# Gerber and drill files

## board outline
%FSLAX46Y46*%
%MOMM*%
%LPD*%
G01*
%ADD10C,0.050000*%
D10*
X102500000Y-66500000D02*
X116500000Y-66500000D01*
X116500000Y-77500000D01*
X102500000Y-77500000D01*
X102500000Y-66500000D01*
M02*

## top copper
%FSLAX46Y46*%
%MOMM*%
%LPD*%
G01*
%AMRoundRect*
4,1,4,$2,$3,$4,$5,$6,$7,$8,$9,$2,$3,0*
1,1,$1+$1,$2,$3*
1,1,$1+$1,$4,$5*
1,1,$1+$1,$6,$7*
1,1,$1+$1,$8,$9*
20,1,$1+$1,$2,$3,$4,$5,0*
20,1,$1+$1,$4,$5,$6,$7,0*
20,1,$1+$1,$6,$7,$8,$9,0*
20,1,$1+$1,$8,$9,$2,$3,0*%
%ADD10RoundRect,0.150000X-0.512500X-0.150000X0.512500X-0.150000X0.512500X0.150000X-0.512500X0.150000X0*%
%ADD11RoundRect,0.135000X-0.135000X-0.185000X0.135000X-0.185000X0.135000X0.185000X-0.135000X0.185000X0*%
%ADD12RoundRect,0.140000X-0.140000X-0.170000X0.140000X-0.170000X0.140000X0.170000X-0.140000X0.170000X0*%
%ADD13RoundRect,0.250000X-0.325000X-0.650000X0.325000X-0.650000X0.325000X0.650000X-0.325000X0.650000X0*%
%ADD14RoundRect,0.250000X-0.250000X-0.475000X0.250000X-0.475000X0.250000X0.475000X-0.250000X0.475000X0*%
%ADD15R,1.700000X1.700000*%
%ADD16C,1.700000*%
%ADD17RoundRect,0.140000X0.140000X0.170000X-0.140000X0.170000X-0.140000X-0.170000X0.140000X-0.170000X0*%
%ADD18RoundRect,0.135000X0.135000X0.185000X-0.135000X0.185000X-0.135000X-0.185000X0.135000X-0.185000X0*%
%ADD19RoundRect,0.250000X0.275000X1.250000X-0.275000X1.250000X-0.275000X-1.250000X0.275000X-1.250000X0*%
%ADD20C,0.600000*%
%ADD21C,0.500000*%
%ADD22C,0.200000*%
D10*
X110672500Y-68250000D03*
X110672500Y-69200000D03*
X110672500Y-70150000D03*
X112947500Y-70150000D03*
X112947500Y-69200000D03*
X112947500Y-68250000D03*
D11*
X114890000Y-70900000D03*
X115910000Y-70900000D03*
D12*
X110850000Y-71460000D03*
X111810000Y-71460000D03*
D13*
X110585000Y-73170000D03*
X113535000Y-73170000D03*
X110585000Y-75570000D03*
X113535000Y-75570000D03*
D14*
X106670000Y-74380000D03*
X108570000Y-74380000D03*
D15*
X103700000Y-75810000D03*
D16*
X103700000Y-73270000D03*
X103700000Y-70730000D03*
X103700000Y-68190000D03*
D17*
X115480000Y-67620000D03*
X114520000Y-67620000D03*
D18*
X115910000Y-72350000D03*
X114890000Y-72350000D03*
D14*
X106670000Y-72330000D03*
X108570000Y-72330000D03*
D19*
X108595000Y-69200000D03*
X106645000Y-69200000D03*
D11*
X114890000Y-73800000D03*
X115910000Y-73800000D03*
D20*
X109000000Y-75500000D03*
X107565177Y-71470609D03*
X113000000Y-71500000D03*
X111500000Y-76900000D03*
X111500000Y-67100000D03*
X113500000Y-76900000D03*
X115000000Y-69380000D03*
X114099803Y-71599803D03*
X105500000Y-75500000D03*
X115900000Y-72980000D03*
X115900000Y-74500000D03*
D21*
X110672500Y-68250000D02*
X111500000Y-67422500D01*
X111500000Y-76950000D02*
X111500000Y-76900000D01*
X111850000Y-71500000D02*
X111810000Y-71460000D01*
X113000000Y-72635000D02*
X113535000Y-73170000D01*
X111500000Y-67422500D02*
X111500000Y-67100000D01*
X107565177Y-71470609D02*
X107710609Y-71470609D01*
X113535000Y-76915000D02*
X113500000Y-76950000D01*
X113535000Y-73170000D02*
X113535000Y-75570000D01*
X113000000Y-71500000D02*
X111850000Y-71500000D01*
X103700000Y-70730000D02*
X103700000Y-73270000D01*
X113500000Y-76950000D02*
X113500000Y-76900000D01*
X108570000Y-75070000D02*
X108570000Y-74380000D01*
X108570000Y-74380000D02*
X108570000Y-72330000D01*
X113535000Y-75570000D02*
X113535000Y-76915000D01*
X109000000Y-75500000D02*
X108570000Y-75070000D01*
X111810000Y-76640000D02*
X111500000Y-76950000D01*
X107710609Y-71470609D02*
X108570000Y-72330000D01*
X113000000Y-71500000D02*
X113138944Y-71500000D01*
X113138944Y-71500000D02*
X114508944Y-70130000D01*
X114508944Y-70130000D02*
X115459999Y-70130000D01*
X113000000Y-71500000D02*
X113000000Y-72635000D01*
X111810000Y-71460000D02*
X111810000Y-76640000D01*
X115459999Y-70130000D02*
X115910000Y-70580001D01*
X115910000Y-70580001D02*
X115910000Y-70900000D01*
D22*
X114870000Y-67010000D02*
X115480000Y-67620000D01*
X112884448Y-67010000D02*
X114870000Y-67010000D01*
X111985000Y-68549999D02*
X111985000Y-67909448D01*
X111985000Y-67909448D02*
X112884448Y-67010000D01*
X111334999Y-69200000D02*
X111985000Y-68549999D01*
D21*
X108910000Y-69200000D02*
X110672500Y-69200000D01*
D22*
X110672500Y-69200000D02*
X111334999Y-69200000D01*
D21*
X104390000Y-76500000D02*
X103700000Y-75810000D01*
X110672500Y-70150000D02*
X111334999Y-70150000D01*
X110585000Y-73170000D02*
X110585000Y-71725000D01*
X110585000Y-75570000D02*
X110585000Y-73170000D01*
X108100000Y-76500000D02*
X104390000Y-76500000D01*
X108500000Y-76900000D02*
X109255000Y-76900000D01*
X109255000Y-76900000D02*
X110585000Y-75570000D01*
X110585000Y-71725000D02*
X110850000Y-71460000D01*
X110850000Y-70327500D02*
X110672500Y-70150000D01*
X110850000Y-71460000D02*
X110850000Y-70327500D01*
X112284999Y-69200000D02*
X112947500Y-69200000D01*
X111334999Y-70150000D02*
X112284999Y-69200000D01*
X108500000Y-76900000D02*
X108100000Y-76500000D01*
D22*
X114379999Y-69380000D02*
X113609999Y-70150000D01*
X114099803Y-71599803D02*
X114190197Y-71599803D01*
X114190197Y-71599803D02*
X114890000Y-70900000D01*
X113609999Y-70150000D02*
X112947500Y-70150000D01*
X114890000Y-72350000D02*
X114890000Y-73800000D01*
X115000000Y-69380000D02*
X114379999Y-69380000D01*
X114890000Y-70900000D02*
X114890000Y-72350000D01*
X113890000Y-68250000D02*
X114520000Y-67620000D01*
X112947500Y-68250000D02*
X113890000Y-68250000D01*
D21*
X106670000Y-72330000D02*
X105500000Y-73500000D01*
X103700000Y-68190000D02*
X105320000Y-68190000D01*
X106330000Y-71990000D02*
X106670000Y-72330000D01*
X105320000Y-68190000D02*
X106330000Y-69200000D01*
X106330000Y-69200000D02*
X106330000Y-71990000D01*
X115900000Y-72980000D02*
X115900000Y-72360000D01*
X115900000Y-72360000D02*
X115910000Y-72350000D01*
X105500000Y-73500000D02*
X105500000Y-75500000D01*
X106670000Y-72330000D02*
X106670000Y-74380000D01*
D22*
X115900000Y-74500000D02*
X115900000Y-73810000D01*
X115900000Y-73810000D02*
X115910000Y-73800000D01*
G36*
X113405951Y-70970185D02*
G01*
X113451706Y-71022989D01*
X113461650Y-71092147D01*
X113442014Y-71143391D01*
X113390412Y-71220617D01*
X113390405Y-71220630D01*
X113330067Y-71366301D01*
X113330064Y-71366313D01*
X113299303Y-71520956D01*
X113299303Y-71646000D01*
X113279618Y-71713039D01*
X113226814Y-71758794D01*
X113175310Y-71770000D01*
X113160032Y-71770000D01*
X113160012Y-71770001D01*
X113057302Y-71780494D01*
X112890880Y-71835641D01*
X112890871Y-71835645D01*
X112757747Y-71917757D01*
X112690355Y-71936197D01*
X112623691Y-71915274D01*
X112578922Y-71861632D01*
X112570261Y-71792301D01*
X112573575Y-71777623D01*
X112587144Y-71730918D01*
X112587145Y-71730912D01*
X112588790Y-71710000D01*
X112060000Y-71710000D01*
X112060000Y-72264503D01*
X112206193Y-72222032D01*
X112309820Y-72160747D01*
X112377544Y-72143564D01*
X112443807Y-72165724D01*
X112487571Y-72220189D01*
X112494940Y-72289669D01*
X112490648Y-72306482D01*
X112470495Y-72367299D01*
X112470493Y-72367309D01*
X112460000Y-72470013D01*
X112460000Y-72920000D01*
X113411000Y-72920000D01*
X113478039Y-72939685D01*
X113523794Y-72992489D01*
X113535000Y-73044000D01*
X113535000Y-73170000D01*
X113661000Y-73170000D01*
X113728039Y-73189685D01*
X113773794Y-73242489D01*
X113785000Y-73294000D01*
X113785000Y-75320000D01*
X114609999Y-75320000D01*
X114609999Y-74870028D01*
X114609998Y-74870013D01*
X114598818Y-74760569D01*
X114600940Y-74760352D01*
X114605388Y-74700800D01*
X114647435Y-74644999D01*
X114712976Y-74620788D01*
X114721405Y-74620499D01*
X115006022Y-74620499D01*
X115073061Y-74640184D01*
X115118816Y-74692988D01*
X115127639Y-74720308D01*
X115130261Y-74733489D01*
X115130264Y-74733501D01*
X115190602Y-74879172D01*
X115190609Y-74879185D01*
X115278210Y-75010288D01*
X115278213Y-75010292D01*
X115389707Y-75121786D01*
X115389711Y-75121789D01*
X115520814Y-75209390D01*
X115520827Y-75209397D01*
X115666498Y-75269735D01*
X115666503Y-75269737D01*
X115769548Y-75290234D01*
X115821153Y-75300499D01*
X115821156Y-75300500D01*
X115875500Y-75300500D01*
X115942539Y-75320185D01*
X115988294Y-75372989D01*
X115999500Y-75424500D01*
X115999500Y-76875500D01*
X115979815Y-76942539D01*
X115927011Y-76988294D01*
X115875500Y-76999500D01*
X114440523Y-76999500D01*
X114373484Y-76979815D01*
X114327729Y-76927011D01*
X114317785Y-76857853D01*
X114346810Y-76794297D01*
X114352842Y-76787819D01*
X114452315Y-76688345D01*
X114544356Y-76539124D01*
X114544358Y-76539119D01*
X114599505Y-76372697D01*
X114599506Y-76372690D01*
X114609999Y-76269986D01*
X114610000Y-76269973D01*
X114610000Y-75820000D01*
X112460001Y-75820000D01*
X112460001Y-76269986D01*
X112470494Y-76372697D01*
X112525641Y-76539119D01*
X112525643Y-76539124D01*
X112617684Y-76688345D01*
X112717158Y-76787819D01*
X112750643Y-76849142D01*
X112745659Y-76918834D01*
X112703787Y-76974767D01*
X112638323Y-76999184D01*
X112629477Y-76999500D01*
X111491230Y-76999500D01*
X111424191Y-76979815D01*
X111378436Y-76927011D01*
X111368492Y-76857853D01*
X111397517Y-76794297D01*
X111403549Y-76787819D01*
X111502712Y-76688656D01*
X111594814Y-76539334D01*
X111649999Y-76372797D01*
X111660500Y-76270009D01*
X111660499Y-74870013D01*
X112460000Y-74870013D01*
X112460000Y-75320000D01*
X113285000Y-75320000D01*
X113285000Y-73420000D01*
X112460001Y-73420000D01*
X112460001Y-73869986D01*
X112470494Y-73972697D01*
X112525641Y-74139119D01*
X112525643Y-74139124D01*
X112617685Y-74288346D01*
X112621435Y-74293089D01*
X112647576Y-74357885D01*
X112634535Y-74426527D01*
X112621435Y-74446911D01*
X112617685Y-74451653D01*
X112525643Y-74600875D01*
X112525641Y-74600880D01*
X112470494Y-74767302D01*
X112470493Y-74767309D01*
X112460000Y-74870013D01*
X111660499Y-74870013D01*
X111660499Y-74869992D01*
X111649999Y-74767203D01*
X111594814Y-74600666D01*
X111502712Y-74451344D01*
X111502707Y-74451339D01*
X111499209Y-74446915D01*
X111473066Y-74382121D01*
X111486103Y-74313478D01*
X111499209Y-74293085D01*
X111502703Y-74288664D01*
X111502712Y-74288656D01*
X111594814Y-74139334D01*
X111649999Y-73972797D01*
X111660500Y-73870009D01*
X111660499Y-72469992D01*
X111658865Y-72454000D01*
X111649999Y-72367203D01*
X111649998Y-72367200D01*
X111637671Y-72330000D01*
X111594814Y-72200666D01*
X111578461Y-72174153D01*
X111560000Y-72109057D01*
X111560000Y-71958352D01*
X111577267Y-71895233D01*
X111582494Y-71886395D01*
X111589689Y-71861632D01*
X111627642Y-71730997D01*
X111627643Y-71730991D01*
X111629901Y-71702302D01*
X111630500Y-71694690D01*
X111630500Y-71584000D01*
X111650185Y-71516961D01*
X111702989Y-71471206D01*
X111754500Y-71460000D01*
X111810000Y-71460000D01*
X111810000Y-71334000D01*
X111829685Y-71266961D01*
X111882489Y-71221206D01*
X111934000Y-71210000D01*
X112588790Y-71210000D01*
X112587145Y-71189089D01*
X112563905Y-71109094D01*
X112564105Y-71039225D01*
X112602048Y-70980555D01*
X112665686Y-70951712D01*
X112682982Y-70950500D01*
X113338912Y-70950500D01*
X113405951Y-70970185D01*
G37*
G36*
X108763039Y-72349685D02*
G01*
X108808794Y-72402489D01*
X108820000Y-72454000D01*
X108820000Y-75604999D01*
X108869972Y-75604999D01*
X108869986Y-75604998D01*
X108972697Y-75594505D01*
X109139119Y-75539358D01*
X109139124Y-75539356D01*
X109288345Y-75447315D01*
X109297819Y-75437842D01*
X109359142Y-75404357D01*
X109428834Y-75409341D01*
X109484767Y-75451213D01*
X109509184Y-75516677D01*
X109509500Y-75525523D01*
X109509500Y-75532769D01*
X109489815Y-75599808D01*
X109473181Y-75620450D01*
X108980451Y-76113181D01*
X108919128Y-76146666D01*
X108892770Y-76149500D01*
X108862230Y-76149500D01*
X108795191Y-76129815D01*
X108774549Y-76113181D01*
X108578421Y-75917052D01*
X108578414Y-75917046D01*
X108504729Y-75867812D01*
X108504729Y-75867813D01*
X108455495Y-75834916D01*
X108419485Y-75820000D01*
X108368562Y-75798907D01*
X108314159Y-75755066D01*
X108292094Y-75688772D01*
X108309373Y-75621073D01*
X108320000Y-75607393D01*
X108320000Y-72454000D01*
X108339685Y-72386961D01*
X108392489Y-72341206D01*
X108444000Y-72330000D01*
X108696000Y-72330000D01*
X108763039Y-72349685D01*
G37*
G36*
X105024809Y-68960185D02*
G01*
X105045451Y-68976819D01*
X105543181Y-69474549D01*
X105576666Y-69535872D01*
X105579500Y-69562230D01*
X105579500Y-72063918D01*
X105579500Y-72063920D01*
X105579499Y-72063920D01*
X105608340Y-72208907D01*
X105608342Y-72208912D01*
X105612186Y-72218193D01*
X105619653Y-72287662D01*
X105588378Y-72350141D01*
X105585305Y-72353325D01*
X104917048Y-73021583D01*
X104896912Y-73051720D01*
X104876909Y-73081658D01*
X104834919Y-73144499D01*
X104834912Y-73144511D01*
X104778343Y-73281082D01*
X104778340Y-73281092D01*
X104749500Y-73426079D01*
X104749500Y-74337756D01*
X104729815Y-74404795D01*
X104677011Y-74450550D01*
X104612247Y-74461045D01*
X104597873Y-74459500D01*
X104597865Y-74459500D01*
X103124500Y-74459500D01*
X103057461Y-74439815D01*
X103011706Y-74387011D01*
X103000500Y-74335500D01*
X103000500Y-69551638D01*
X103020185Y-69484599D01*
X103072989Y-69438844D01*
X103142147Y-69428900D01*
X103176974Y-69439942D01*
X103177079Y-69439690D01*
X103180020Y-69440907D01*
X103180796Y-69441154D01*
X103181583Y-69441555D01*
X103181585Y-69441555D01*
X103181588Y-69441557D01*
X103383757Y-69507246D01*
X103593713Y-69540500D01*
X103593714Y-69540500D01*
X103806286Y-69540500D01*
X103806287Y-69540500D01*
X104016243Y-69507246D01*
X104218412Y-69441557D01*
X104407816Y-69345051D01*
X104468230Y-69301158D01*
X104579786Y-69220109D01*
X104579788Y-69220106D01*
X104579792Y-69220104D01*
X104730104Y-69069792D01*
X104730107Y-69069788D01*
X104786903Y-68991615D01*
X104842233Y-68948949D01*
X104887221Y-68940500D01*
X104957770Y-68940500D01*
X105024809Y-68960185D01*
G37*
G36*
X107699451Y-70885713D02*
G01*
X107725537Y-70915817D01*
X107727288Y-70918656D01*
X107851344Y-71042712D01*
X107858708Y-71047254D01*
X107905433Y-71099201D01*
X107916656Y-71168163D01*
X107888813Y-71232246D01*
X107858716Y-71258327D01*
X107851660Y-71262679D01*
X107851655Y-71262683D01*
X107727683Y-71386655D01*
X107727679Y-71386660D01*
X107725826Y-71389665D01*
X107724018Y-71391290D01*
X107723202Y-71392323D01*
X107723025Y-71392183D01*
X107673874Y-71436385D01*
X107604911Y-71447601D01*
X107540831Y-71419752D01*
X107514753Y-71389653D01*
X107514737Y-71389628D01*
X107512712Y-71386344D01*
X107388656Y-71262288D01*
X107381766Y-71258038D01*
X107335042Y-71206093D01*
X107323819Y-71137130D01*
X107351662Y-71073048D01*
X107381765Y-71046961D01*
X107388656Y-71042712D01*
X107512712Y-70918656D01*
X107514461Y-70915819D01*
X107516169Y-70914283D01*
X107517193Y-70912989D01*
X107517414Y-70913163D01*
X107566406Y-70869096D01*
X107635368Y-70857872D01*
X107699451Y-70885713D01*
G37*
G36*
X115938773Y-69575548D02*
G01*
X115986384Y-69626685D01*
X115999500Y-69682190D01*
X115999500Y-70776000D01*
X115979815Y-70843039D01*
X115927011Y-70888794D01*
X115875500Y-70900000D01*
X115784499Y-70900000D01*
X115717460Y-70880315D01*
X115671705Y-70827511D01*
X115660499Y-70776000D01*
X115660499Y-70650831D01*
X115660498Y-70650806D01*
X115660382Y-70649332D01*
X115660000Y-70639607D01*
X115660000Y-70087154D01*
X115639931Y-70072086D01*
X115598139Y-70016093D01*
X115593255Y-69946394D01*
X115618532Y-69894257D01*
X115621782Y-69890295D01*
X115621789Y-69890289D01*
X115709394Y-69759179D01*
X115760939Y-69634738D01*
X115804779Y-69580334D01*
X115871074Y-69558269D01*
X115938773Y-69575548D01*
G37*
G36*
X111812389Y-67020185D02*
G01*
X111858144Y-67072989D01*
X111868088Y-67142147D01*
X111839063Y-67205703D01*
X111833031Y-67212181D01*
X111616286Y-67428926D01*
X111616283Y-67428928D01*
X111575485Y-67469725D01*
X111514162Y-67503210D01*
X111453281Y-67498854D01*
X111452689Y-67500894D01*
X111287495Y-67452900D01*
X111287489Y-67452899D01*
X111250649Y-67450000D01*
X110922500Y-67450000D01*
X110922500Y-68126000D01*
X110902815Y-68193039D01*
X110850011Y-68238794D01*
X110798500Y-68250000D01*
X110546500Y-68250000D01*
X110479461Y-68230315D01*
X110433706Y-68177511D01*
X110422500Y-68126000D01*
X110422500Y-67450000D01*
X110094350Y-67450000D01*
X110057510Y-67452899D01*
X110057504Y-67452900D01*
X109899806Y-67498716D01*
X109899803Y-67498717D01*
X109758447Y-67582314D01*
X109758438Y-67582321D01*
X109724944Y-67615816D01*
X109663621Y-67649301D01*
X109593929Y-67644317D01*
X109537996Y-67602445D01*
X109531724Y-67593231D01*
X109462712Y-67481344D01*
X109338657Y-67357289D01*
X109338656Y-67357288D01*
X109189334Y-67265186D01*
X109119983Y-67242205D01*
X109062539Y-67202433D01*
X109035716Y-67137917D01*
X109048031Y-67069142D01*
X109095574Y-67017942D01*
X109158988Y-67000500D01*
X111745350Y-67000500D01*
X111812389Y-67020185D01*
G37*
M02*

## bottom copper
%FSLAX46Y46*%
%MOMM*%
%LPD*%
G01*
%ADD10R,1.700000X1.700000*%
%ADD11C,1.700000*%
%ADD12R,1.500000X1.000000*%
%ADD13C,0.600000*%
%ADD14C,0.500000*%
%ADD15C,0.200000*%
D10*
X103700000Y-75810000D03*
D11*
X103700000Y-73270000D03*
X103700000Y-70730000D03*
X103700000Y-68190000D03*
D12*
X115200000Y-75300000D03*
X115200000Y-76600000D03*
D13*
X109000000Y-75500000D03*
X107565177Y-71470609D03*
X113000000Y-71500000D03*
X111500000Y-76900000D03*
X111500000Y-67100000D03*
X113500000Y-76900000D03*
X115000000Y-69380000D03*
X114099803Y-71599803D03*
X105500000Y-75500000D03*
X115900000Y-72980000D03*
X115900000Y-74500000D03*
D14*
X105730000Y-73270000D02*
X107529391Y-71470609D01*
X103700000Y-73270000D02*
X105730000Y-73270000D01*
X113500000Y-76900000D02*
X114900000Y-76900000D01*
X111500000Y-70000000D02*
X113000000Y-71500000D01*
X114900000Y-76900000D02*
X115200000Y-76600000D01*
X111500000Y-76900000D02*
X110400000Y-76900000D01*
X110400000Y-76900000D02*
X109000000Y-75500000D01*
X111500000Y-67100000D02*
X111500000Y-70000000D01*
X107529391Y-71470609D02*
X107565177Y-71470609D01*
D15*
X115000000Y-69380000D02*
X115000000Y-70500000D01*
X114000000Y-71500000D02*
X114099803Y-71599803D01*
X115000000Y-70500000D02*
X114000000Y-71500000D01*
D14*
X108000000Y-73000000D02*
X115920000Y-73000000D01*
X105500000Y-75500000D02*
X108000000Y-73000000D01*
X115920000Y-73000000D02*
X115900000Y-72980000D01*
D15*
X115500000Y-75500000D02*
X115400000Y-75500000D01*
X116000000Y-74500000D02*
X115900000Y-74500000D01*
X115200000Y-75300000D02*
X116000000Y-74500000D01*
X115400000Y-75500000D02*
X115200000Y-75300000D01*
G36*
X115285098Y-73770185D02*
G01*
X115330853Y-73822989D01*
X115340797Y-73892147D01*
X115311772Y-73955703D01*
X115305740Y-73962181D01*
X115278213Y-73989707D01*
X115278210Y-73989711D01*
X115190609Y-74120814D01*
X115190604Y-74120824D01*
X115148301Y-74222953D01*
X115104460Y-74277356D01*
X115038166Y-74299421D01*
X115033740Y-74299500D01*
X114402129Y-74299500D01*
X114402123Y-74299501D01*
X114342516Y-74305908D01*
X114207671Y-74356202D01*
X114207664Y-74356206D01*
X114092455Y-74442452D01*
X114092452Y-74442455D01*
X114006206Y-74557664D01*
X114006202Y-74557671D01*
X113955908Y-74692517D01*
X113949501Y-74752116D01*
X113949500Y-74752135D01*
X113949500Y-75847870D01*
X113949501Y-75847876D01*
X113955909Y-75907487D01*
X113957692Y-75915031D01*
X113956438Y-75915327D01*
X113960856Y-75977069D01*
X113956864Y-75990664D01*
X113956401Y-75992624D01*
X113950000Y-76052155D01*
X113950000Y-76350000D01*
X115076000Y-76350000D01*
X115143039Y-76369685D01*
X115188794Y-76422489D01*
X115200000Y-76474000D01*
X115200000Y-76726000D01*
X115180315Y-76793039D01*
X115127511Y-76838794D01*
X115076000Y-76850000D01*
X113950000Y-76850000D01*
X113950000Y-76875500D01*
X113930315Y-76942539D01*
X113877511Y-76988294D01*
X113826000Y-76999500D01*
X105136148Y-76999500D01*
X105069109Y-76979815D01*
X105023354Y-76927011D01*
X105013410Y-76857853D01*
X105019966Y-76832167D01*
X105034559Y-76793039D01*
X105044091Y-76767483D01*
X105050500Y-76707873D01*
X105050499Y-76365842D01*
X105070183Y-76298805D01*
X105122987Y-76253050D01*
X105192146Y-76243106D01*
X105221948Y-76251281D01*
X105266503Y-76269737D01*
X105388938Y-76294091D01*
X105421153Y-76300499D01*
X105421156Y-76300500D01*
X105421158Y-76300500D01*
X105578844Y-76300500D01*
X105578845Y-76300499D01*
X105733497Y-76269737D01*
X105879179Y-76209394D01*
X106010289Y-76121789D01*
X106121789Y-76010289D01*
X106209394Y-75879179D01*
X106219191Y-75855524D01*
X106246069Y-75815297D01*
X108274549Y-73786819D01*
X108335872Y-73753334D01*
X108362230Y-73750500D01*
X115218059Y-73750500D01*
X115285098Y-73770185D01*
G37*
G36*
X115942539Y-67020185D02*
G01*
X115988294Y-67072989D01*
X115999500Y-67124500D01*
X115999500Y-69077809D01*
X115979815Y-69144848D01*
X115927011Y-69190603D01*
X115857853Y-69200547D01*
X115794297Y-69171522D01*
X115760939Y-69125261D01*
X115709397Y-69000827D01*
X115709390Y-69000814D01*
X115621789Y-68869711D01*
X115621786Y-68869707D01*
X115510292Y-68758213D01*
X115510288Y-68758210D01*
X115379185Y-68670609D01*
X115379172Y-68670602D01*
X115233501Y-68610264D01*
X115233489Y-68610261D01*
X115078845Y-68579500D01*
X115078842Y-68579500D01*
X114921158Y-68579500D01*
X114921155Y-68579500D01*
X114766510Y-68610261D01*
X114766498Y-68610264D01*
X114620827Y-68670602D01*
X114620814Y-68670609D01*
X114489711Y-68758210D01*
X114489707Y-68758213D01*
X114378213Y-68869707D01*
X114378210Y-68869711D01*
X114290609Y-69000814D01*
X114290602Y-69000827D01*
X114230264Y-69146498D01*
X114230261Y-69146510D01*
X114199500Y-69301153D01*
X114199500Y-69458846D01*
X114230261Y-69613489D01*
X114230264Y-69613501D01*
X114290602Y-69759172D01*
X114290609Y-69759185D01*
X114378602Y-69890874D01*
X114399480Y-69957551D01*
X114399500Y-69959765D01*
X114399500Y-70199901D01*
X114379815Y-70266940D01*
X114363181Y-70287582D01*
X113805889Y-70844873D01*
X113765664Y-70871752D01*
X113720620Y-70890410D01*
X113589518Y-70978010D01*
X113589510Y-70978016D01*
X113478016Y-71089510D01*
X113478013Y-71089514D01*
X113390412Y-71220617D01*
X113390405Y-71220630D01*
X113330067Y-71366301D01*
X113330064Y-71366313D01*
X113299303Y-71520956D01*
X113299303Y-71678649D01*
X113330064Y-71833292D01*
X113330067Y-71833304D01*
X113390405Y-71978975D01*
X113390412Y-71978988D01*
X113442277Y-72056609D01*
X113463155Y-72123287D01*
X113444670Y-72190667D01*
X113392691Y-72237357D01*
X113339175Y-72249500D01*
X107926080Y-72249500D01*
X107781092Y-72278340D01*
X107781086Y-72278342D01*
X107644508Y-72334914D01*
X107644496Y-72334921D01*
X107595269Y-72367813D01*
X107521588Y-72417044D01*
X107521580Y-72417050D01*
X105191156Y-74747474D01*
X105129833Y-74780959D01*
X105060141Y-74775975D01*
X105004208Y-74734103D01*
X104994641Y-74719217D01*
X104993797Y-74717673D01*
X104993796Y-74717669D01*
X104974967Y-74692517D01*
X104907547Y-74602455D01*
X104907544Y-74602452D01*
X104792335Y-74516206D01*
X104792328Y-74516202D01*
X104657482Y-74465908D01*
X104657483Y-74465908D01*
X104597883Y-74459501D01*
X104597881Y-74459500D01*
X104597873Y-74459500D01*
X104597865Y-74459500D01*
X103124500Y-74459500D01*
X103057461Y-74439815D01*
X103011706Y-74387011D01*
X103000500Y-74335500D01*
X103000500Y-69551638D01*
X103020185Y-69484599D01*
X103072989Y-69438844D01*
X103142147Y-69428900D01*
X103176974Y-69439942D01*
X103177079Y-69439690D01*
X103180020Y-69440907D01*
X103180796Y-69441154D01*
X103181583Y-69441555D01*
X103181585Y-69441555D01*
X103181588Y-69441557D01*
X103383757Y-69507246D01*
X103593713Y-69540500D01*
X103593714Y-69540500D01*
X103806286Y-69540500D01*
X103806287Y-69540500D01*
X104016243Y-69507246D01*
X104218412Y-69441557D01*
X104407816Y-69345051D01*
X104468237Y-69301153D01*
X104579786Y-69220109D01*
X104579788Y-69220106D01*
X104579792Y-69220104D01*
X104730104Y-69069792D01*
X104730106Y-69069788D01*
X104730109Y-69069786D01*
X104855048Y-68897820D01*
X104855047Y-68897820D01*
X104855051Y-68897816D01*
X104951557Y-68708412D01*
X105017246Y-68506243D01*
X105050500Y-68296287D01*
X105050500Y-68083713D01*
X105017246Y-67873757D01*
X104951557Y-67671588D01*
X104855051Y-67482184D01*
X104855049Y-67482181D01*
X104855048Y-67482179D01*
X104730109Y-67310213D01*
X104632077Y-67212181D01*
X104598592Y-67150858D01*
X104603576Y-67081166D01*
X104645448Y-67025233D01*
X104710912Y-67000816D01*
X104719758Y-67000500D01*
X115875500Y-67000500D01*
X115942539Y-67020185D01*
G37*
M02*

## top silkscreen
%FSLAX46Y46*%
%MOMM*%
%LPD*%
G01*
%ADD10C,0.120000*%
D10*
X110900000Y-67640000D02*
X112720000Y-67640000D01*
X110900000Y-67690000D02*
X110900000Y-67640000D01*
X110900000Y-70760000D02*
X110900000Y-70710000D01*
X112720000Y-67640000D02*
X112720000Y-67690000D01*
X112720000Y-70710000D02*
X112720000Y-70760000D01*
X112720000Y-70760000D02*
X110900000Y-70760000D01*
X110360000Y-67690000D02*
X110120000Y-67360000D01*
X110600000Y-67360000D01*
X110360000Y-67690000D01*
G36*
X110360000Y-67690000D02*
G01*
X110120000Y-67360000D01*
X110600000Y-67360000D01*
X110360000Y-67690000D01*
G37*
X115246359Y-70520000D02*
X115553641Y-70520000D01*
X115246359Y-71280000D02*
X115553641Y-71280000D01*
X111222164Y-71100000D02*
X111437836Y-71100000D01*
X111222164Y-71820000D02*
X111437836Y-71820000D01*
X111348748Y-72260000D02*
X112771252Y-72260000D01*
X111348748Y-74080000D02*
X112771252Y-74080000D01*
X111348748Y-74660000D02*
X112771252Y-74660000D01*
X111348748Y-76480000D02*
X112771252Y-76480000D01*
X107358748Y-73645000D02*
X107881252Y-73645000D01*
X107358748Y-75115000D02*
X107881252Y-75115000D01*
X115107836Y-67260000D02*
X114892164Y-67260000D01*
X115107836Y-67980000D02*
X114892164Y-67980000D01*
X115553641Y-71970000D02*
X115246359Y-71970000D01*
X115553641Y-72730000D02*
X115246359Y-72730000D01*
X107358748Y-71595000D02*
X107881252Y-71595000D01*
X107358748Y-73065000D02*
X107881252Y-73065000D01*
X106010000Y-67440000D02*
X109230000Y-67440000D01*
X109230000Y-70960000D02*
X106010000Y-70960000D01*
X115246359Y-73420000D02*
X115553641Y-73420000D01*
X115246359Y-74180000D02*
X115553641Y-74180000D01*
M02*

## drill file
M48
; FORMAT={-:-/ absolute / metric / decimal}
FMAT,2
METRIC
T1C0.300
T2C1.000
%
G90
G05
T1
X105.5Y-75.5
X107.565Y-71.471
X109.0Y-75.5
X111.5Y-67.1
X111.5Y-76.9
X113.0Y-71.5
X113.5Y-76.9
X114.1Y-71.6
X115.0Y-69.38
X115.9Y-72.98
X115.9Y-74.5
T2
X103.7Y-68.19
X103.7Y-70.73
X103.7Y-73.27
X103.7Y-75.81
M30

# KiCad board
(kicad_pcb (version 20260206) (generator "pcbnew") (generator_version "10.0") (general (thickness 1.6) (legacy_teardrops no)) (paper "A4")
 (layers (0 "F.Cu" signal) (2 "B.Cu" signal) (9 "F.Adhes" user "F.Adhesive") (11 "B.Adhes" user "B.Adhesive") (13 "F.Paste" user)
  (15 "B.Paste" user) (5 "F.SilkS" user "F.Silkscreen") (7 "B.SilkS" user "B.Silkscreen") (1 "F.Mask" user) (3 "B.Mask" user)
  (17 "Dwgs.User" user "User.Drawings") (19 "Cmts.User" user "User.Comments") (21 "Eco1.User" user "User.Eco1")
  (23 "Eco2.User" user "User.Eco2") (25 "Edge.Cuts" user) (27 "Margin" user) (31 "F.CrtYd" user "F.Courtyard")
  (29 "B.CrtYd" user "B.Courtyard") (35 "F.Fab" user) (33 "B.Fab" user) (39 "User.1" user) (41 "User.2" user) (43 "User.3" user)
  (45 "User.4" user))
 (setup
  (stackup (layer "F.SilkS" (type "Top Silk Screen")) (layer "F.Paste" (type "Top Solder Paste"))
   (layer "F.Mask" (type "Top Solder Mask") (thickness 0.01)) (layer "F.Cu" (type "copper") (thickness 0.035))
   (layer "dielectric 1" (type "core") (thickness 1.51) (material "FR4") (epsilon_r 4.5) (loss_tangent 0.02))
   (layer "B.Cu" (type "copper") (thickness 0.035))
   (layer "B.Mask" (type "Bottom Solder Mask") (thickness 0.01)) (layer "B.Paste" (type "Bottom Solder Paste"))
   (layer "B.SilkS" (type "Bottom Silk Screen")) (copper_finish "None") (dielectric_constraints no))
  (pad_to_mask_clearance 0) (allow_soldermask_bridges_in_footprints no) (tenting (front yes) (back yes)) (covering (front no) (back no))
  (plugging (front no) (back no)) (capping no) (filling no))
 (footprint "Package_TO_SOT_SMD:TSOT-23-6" (layer "F.Cu") (at 111.81 69.2)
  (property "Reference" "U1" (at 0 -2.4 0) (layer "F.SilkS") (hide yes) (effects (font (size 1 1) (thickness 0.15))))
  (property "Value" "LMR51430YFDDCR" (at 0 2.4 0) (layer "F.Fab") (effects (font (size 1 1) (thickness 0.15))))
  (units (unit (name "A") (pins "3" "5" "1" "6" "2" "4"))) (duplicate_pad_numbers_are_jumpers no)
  (fp_line (start -0.91 -1.56) (end 0.91 -1.56) (stroke (width 0.12) (type solid)) (layer "F.SilkS"))
  (fp_line (start -0.91 -1.51) (end -0.91 -1.56) (stroke (width 0.12) (type solid)) (layer "F.SilkS"))
  (fp_line (start -0.91 1.56) (end -0.91 1.51) (stroke (width 0.12) (type solid)) (layer "F.SilkS"))
  (fp_line (start 0.91 -1.56) (end 0.91 -1.51) (stroke (width 0.12) (type solid)) (layer "F.SilkS"))
  (fp_line (start 0.91 1.51) (end 0.91 1.56) (stroke (width 0.12) (type solid)) (layer "F.SilkS"))
  (fp_line (start 0.91 1.56) (end -0.91 1.56) (stroke (width 0.12) (type solid)) (layer "F.SilkS"))
  (fp_poly (pts (xy -1.45 -1.51) (xy -1.69 -1.84) (xy -1.21 -1.84)) (stroke (width 0.12) (type solid)) (fill yes) (layer "F.SilkS"))
  (pad "1" smd roundrect (at -1.1375 -0.95) (size 1.325 0.6) (layers "F.Cu" "F.Mask" "F.Paste") (roundrect_rratio 0.25) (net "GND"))
  (pad "2" smd roundrect (at -1.1375 0) (size 1.325 0.6) (layers "F.Cu" "F.Mask" "F.Paste") (roundrect_rratio 0.25) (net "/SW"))
  (pad "3" smd roundrect (at -1.1375 0.95) (size 1.325 0.6) (layers "F.Cu" "F.Mask" "F.Paste") (roundrect_rratio 0.25) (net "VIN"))
  (pad "4" smd roundrect (at 1.1375 0.95) (size 1.325 0.6) (layers "F.Cu" "F.Mask" "F.Paste") (roundrect_rratio 0.25) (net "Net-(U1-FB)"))
  (pad "5" smd roundrect (at 1.1375 0) (size 1.325 0.6) (layers "F.Cu" "F.Mask" "F.Paste") (roundrect_rratio 0.25) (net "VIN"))
  (pad "6" smd roundrect (at 1.1375 -0.95) (size 1.325 0.6) (layers "F.Cu" "F.Mask" "F.Paste") (roundrect_rratio 0.25) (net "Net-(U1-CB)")))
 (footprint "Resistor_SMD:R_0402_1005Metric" (layer "F.Cu") (at 115.4 70.9)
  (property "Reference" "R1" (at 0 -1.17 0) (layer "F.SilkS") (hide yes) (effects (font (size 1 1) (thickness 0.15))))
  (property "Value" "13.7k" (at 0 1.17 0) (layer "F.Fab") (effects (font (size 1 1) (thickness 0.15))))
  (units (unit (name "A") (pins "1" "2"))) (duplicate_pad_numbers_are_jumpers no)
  (fp_line (start -0.153641 -0.38) (end 0.153641 -0.38) (stroke (width 0.12) (type solid)) (layer "F.SilkS"))
  (fp_line (start -0.153641 0.38) (end 0.153641 0.38) (stroke (width 0.12) (type solid)) (layer "F.SilkS"))
  (pad "1" smd roundrect (at -0.51 0) (size 0.54 0.64) (layers "F.Cu" "F.Mask" "F.Paste") (roundrect_rratio 0.25) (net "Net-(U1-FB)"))
  (pad "2" smd roundrect (at 0.51 0) (size 0.54 0.64) (layers "F.Cu" "F.Mask" "F.Paste") (roundrect_rratio 0.25) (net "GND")))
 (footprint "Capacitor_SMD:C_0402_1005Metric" (layer "F.Cu") (at 111.33 71.46)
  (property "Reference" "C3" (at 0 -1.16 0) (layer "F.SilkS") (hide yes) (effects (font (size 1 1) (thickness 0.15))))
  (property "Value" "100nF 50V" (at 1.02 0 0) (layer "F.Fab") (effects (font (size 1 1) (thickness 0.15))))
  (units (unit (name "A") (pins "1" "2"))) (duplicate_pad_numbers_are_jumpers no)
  (fp_line (start -0.107836 -0.36) (end 0.107836 -0.36) (stroke (width 0.12) (type solid)) (layer "F.SilkS"))
  (fp_line (start -0.107836 0.36) (end 0.107836 0.36) (stroke (width 0.12) (type solid)) (layer "F.SilkS"))
  (pad "1" smd roundrect (at -0.48 0) (size 0.56 0.62) (layers "F.Cu" "F.Mask" "F.Paste") (roundrect_rratio 0.25) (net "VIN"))
  (pad "2" smd roundrect (at 0.48 0) (size 0.56 0.62) (layers "F.Cu" "F.Mask" "F.Paste") (roundrect_rratio 0.25) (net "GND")))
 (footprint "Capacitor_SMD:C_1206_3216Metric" (layer "F.Cu") (at 112.06 73.17)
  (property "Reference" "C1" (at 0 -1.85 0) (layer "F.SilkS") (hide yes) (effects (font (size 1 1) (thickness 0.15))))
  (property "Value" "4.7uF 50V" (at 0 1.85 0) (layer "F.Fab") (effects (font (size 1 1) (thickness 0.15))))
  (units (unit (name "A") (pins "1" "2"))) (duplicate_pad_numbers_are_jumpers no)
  (fp_line (start -0.711252 -0.91) (end 0.711252 -0.91) (stroke (width 0.12) (type solid)) (layer "F.SilkS"))
  (fp_line (start -0.711252 0.91) (end 0.711252 0.91) (stroke (width 0.12) (type solid)) (layer "F.SilkS"))
  (pad "1" smd roundrect (at -1.475 0) (size 1.15 1.8) (layers "F.Cu" "F.Mask" "F.Paste") (roundrect_rratio 0.217391) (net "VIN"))
  (pad "2" smd roundrect (at 1.475 0) (size 1.15 1.8) (layers "F.Cu" "F.Mask" "F.Paste") (roundrect_rratio 0.217391) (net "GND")))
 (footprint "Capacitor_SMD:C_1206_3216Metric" (layer "F.Cu") (at 112.06 75.57)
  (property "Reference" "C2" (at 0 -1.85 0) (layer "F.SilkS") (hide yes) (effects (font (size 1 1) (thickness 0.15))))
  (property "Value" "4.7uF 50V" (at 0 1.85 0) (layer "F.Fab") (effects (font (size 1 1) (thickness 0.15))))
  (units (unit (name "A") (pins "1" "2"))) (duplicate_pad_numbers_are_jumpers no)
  (fp_line (start -0.711252 -0.91) (end 0.711252 -0.91) (stroke (width 0.12) (type solid)) (layer "F.SilkS"))
  (fp_line (start -0.711252 0.91) (end 0.711252 0.91) (stroke (width 0.12) (type solid)) (layer "F.SilkS"))
  (pad "1" smd roundrect (at -1.475 0) (size 1.15 1.8) (layers "F.Cu" "F.Mask" "F.Paste") (roundrect_rratio 0.217391) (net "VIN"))
  (pad "2" smd roundrect (at 1.475 0) (size 1.15 1.8) (layers "F.Cu" "F.Mask" "F.Paste") (roundrect_rratio 0.217391) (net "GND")))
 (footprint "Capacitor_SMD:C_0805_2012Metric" (layer "F.Cu") (at 107.62 74.38)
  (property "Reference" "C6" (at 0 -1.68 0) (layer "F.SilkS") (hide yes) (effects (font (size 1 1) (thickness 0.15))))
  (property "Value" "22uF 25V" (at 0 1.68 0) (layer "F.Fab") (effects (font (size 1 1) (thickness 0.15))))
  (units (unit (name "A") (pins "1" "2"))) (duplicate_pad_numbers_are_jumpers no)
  (fp_line (start -0.261252 -0.735) (end 0.261252 -0.735) (stroke (width 0.12) (type solid)) (layer "F.SilkS"))
  (fp_line (start -0.261252 0.735) (end 0.261252 0.735) (stroke (width 0.12) (type solid)) (layer "F.SilkS"))
  (pad "1" smd roundrect (at -0.95 0) (size 1 1.45) (layers "F.Cu" "F.Mask" "F.Paste") (roundrect_rratio 0.25) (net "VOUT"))
  (pad "2" smd roundrect (at 0.95 0) (size 1 1.45) (layers "F.Cu" "F.Mask" "F.Paste") (roundrect_rratio 0.25) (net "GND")))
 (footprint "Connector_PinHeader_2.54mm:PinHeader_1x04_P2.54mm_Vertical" (layer "F.Cu") (at 103.7 75.81 180)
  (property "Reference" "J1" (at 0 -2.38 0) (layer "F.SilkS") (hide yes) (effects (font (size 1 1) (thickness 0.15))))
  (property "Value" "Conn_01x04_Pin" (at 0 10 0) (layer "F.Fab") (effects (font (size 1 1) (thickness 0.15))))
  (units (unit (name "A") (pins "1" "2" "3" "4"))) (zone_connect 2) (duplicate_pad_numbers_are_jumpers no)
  (pad "1" thru_hole rect (at 0 0 180) (size 1.7 1.7) (drill 1) (layers "*.Cu" "*.Mask") (remove_unused_layers no) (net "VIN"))
  (pad "2" thru_hole circle (at 0 2.54 180) (size 1.7 1.7) (drill 1) (layers "*.Cu" "*.Mask") (remove_unused_layers no) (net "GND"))
  (pad "3" thru_hole circle (at 0 5.08 180) (size 1.7 1.7) (drill 1) (layers "*.Cu" "*.Mask") (remove_unused_layers no) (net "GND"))
  (pad "4" thru_hole circle (at 0 7.62 180) (size 1.7 1.7) (drill 1) (layers "*.Cu" "*.Mask") (remove_unused_layers no) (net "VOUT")))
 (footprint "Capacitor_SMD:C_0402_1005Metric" (layer "F.Cu") (at 115 67.62 180)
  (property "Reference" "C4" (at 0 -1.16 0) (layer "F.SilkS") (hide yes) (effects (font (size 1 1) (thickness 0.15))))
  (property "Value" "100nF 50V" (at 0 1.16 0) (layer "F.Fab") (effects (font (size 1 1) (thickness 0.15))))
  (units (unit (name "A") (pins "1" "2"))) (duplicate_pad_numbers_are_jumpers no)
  (fp_line (start -0.107836 0.36) (end 0.107836 0.36) (stroke (width 0.12) (type solid)) (layer "F.SilkS"))
  (fp_line (start -0.107836 -0.36) (end 0.107836 -0.36) (stroke (width 0.12) (type solid)) (layer "F.SilkS"))
  (pad "1" smd roundrect (at -0.48 0 180) (size 0.56 0.62) (layers "F.Cu" "F.Mask" "F.Paste") (roundrect_rratio 0.25) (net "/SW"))
  (pad "2" smd roundrect (at 0.48 0 180) (size 0.56 0.62) (layers "F.Cu" "F.Mask" "F.Paste") (roundrect_rratio 0.25) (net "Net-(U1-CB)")))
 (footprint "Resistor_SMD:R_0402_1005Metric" (layer "F.Cu") (at 115.4 72.35 180)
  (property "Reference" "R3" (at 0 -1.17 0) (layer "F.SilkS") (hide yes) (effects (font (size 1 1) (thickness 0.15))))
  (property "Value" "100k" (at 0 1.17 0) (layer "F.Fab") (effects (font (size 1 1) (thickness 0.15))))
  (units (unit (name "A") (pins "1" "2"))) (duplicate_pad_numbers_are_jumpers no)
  (fp_line (start -0.153641 0.38) (end 0.153641 0.38) (stroke (width 0.12) (type solid)) (layer "F.SilkS"))
  (fp_line (start -0.153641 -0.38) (end 0.153641 -0.38) (stroke (width 0.12) (type solid)) (layer "F.SilkS"))
  (pad "1" smd roundrect (at -0.51 0 180) (size 0.54 0.64) (layers "F.Cu" "F.Mask" "F.Paste") (roundrect_rratio 0.25) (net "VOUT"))
  (pad "2" smd roundrect (at 0.51 0 180) (size 0.54 0.64) (layers "F.Cu" "F.Mask" "F.Paste") (roundrect_rratio 0.25) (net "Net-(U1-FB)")))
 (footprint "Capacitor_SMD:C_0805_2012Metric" (layer "F.Cu") (at 107.62 72.33)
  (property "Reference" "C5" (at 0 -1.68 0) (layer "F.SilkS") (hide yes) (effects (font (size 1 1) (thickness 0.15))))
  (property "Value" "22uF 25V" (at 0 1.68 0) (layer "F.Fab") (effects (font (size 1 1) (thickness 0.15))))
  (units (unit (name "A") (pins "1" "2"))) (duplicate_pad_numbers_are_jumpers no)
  (fp_line (start -0.261252 -0.735) (end 0.261252 -0.735) (stroke (width 0.12) (type solid)) (layer "F.SilkS"))
  (fp_line (start -0.261252 0.735) (end 0.261252 0.735) (stroke (width 0.12) (type solid)) (layer "F.SilkS"))
  (pad "1" smd roundrect (at -0.95 0) (size 1 1.45) (layers "F.Cu" "F.Mask" "F.Paste") (roundrect_rratio 0.25) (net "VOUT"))
  (pad "2" smd roundrect (at 0.95 0) (size 1 1.45) (layers "F.Cu" "F.Mask" "F.Paste") (roundrect_rratio 0.25) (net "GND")))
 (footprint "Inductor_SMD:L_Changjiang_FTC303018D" (layer "F.Cu") (at 107.62 69.2 180)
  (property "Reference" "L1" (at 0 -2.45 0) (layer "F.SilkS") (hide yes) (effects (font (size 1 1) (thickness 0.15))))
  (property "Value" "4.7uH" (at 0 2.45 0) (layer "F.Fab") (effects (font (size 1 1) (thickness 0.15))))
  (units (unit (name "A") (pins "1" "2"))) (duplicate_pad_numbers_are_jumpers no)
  (fp_line (start 1.61 1.76) (end -1.61 1.76) (stroke (width 0.12) (type solid)) (layer "F.SilkS"))
  (fp_line (start -1.61 -1.76) (end 1.61 -1.76) (stroke (width 0.12) (type solid)) (layer "F.SilkS"))
  (pad "1" smd roundrect (at -0.975 0 180) (size 1.05 3) (layers "F.Cu" "F.Mask" "F.Paste") (roundrect_rratio 0.238095) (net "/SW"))
  (pad "2" smd roundrect (at 0.975 0 180) (size 1.05 3) (layers "F.Cu" "F.Mask" "F.Paste") (roundrect_rratio 0.238095) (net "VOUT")))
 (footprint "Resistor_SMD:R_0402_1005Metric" (layer "F.Cu") (at 115.4 73.8)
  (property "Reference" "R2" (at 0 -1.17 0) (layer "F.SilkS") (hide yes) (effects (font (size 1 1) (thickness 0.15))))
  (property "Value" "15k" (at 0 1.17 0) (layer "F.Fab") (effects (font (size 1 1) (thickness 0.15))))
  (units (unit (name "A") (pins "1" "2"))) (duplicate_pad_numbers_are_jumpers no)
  (fp_line (start -0.153641 -0.38) (end 0.153641 -0.38) (stroke (width 0.12) (type solid)) (layer "F.SilkS"))
  (fp_line (start -0.153641 0.38) (end 0.153641 0.38) (stroke (width 0.12) (type solid)) (layer "F.SilkS"))
  (pad "1" smd roundrect (at -0.51 0) (size 0.54 0.64) (layers "F.Cu" "F.Mask" "F.Paste") (roundrect_rratio 0.25) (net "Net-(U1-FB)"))
  (pad "2" smd roundrect (at 0.51 0) (size 0.54 0.64) (layers "F.Cu" "F.Mask" "F.Paste") (roundrect_rratio 0.25) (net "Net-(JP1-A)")))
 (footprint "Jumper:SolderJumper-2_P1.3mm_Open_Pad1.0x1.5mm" (layer "B.Cu") (at 115.2 75.95 -90)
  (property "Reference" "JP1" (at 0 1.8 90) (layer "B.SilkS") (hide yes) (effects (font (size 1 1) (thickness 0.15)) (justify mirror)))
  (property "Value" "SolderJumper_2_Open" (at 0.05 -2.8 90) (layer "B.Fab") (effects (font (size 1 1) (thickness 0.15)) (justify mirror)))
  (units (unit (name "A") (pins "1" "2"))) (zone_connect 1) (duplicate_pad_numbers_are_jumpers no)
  (pad "1" smd rect (at -0.65 0 270) (size 1 1.5) (layers "B.Cu" "B.Mask") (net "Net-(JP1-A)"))
  (pad "2" smd rect (at 0.65 0 270) (size 1 1.5) (layers "B.Cu" "B.Mask") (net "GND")))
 (gr_rect (start 102.5 66.5) (end 116.5 77.5) (stroke (width 0.05) (type default)) (fill no) (layer "Edge.Cuts"))
 (segment (start 110.6725 68.25) (end 111.5 67.4225) (width 0.5) (layer "F.Cu") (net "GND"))
 (segment (start 111.5 76.95) (end 111.5 76.9) (width 0.5) (layer "F.Cu") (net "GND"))
 (segment (start 111.85 71.5) (end 111.81 71.46) (width 0.5) (layer "F.Cu") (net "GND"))
 (segment (start 113 72.635) (end 113.535 73.17) (width 0.5) (layer "F.Cu") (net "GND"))
 (segment (start 111.5 67.4225) (end 111.5 67.1) (width 0.5) (layer "F.Cu") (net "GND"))
 (segment (start 107.565177 71.470609) (end 107.710609 71.470609) (width 0.5) (layer "F.Cu") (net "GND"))
 (segment (start 113.535 76.915) (end 113.5 76.95) (width 0.5) (layer "F.Cu") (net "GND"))
 (segment (start 113.535 73.17) (end 113.535 75.57) (width 0.5) (layer "F.Cu") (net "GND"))
 (segment (start 113 71.5) (end 111.85 71.5) (width 0.5) (layer "F.Cu") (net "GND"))
 (segment (start 103.7 70.73) (end 103.7 73.27) (width 0.5) (layer "F.Cu") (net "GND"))
 (segment (start 113.5 76.95) (end 113.5 76.9) (width 0.5) (layer "F.Cu") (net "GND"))
 (segment (start 108.57 75.07) (end 108.57 74.38) (width 0.5) (layer "F.Cu") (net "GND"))
 (segment (start 108.57 74.38) (end 108.57 72.33) (width 0.5) (layer "F.Cu") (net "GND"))
 (segment (start 113.535 75.57) (end 113.535 76.915) (width 0.5) (layer "F.Cu") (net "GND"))
 (segment (start 109 75.5) (end 108.57 75.07) (width 0.5) (layer "F.Cu") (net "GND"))
 (segment (start 111.81 76.64) (end 111.5 76.95) (width 0.5) (layer "F.Cu") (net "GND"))
 (segment (start 107.710609 71.470609) (end 108.57 72.33) (width 0.5) (layer "F.Cu") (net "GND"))
 (segment (start 113 71.5) (end 113.138944 71.5) (width 0.5) (layer "F.Cu") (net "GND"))
 (segment (start 113.138944 71.5) (end 114.508944 70.13) (width 0.5) (layer "F.Cu") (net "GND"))
 (segment (start 114.508944 70.13) (end 115.459999 70.13) (width 0.5) (layer "F.Cu") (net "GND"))
 (segment (start 113 71.5) (end 113 72.635) (width 0.5) (layer "F.Cu") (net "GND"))
 (segment (start 111.81 71.46) (end 111.81 76.64) (width 0.5) (layer "F.Cu") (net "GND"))
 (segment (start 115.459999 70.13) (end 115.91 70.580001) (width 0.5) (layer "F.Cu") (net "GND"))
 (segment (start 115.91 70.580001) (end 115.91 70.9) (width 0.5) (layer "F.Cu") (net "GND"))
 (via (at 109 75.5) (size 0.6) (drill 0.3) (layers "F.Cu" "B.Cu") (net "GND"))
 (via (at 107.565177 71.470609) (size 0.6) (drill 0.3) (layers "F.Cu" "B.Cu") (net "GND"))
 (via (at 113 71.5) (size 0.6) (drill 0.3) (layers "F.Cu" "B.Cu") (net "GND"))
 (via (at 111.5 76.9) (size 0.6) (drill 0.3) (layers "F.Cu" "B.Cu") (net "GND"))
 (via (at 111.5 67.1) (size 0.6) (drill 0.3) (layers "F.Cu" "B.Cu") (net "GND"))
 (via (at 113.5 76.9) (size 0.6) (drill 0.3) (layers "F.Cu" "B.Cu") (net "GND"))
 (segment (start 105.73 73.27) (end 107.529391 71.470609) (width 0.5) (layer "B.Cu") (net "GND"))
 (segment (start 103.7 73.27) (end 105.73 73.27) (width 0.5) (layer "B.Cu") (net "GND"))
 (segment (start 113.5 76.9) (end 114.9 76.9) (width 0.5) (layer "B.Cu") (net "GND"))
 (segment (start 111.5 70) (end 113 71.5) (width 0.5) (layer "B.Cu") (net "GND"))
 (segment (start 114.9 76.9) (end 115.2 76.6) (width 0.5) (layer "B.Cu") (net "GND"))
 (segment (start 111.5 76.9) (end 110.4 76.9) (width 0.5) (layer "B.Cu") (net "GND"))
 (segment (start 110.4 76.9) (end 109 75.5) (width 0.5) (layer "B.Cu") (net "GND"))
 (segment (start 111.5 67.1) (end 111.5 70) (width 0.5) (layer "B.Cu") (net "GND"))
 (segment (start 107.529391 71.470609) (end 107.565177 71.470609) (width 0.5) (layer "B.Cu") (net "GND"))
 (segment (start 114.87 67.01) (end 115.48 67.62) (width 0.2) (layer "F.Cu") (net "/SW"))
 (segment (start 112.884448 67.01) (end 114.87 67.01) (width 0.2) (layer "F.Cu") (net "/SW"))
 (segment (start 111.985 68.549999) (end 111.985 67.909448) (width 0.2) (layer "F.Cu") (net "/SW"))
 (segment (start 111.985 67.909448) (end 112.884448 67.01) (width 0.2) (layer "F.Cu") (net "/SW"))
 (segment (start 111.334999 69.2) (end 111.985 68.549999) (width 0.2) (layer "F.Cu") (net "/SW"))
 (segment (start 108.91 69.2) (end 110.6725 69.2) (width 0.5) (layer "F.Cu") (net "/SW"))
 (segment (start 110.6725 69.2) (end 111.334999 69.2) (width 0.2) (layer "F.Cu") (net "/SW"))
 (segment (start 104.39 76.5) (end 103.7 75.81) (width 0.5) (layer "F.Cu") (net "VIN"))
 (segment (start 110.6725 70.15) (end 111.334999 70.15) (width 0.5) (layer "F.Cu") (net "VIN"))
 (segment (start 110.585 73.17) (end 110.585 71.725) (width 0.5) (layer "F.Cu") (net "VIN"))
 (segment (start 110.585 75.57) (end 110.585 73.17) (width 0.5) (layer "F.Cu") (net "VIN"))
 (segment (start 108.1 76.5) (end 104.39 76.5) (width 0.5) (layer "F.Cu") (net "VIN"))
 (segment (start 108.5 76.9) (end 109.255 76.9) (width 0.5) (layer "F.Cu") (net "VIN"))
 (segment (start 109.255 76.9) (end 110.585 75.57) (width 0.5) (layer "F.Cu") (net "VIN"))
 (segment (start 110.585 71.725) (end 110.85 71.46) (width 0.5) (layer "F.Cu") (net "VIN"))
 (segment (start 110.85 70.3275) (end 110.6725 70.15) (width 0.5) (layer "F.Cu") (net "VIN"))
 (segment (start 110.85 71.46) (end 110.85 70.3275) (width 0.5) (layer "F.Cu") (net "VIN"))
 (segment (start 112.284999 69.2) (end 112.9475 69.2) (width 0.5) (layer "F.Cu") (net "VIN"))
 (segment (start 111.334999 70.15) (end 112.284999 69.2) (width 0.5) (layer "F.Cu") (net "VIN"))
 (segment (start 108.5 76.9) (end 108.1 76.5) (width 0.5) (layer "F.Cu") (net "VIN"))
 (segment (start 114.379999 69.38) (end 113.609999 70.15) (width 0.2) (layer "F.Cu") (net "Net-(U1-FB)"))
 (segment (start 114.099803 71.599803) (end 114.190197 71.599803) (width 0.2) (layer "F.Cu") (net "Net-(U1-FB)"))
 (segment (start 114.190197 71.599803) (end 114.89 70.9) (width 0.2) (layer "F.Cu") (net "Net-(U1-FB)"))
 (segment (start 113.609999 70.15) (end 112.9475 70.15) (width 0.2) (layer "F.Cu") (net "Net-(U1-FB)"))
 (segment (start 114.89 72.35) (end 114.89 73.8) (width 0.2) (layer "F.Cu") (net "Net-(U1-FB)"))
 (segment (start 115 69.38) (end 114.379999 69.38) (width 0.2) (layer "F.Cu") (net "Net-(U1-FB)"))
 (segment (start 114.89 70.9) (end 114.89 72.35) (width 0.2) (layer "F.Cu") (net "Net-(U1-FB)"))
 (via (at 115 69.38) (size 0.6) (drill 0.3) (layers "F.Cu" "B.Cu") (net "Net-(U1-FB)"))
 (via (at 114.099803 71.599803) (size 0.6) (drill 0.3) (layers "F.Cu" "B.Cu") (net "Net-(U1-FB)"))
 (segment (start 115 69.38) (end 115 70.5) (width 0.2) (layer "B.Cu") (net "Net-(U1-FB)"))
 (segment (start 114 71.5) (end 114.099803 71.599803) (width 0.2) (layer "B.Cu") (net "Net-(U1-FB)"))
 (segment (start 115 70.5) (end 114 71.5) (width 0.2) (layer "B.Cu") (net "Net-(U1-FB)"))
 (segment (start 113.89 68.25) (end 114.52 67.62) (width 0.2) (layer "F.Cu") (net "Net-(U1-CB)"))
 (segment (start 112.9475 68.25) (end 113.89 68.25) (width 0.2) (layer "F.Cu") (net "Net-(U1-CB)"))
 (segment (start 106.67 72.33) (end 105.5 73.5) (width 0.5) (layer "F.Cu") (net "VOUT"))
 (segment (start 103.7 68.19) (end 105.32 68.19) (width 0.5) (layer "F.Cu") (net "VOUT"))
 (segment (start 106.33 71.99) (end 106.67 72.33) (width 0.5) (layer "F.Cu") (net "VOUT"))
 (segment (start 105.32 68.19) (end 106.33 69.2) (width 0.5) (layer "F.Cu") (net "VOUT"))
 (segment (start 106.33 69.2) (end 106.33 71.99) (width 0.5) (layer "F.Cu") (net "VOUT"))
 (segment (start 115.9 72.98) (end 115.9 72.36) (width 0.5) (layer "F.Cu") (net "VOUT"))
 (segment (start 115.9 72.36) (end 115.91 72.35) (width 0.5) (layer "F.Cu") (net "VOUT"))
 (segment (start 105.5 73.5) (end 105.5 75.5) (width 0.5) (layer "F.Cu") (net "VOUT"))
 (segment (start 106.67 72.33) (end 106.67 74.38) (width 0.5) (layer "F.Cu") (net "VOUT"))
 (via (at 105.5 75.5) (size 0.6) (drill 0.3) (layers "F.Cu" "B.Cu") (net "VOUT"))
 (via (at 115.9 72.98) (size 0.6) (drill 0.3) (layers "F.Cu" "B.Cu") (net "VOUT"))
 (segment (start 108 73) (end 115.92 73) (width 0.5) (layer "B.Cu") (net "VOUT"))
 (segment (start 105.5 75.5) (end 108 73) (width 0.5) (layer "B.Cu") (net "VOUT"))
 (segment (start 115.92 73) (end 115.9 72.98) (width 0.5) (layer "B.Cu") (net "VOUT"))
 (segment (start 115.9 74.5) (end 115.9 73.81) (width 0.2) (layer "F.Cu") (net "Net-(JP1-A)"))
 (segment (start 115.9 73.81) (end 115.91 73.8) (width 0.2) (layer "F.Cu") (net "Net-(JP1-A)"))
 (via (at 115.9 74.5) (size 0.6) (drill 0.3) (layers "F.Cu" "B.Cu") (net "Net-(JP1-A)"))
 (segment (start 115.5 75.5) (end 115.4 75.5) (width 0.2) (layer "B.Cu") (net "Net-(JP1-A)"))
 (segment (start 116 74.5) (end 115.9 74.5) (width 0.2) (layer "B.Cu") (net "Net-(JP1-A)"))
 (segment (start 115.2 75.3) (end 116 74.5) (width 0.2) (layer "B.Cu") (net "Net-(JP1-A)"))
 (segment (start 115.4 75.5) (end 115.2 75.3) (width 0.2) (layer "B.Cu") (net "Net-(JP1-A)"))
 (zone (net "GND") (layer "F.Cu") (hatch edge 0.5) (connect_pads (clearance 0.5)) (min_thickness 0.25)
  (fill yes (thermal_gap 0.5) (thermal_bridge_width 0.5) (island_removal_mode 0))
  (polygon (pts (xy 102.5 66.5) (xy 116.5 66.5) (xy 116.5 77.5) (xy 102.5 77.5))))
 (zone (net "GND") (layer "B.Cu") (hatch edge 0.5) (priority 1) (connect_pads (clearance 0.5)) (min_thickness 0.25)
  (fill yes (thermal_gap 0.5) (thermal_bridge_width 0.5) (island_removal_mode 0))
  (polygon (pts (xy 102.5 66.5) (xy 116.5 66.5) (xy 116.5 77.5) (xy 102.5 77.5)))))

